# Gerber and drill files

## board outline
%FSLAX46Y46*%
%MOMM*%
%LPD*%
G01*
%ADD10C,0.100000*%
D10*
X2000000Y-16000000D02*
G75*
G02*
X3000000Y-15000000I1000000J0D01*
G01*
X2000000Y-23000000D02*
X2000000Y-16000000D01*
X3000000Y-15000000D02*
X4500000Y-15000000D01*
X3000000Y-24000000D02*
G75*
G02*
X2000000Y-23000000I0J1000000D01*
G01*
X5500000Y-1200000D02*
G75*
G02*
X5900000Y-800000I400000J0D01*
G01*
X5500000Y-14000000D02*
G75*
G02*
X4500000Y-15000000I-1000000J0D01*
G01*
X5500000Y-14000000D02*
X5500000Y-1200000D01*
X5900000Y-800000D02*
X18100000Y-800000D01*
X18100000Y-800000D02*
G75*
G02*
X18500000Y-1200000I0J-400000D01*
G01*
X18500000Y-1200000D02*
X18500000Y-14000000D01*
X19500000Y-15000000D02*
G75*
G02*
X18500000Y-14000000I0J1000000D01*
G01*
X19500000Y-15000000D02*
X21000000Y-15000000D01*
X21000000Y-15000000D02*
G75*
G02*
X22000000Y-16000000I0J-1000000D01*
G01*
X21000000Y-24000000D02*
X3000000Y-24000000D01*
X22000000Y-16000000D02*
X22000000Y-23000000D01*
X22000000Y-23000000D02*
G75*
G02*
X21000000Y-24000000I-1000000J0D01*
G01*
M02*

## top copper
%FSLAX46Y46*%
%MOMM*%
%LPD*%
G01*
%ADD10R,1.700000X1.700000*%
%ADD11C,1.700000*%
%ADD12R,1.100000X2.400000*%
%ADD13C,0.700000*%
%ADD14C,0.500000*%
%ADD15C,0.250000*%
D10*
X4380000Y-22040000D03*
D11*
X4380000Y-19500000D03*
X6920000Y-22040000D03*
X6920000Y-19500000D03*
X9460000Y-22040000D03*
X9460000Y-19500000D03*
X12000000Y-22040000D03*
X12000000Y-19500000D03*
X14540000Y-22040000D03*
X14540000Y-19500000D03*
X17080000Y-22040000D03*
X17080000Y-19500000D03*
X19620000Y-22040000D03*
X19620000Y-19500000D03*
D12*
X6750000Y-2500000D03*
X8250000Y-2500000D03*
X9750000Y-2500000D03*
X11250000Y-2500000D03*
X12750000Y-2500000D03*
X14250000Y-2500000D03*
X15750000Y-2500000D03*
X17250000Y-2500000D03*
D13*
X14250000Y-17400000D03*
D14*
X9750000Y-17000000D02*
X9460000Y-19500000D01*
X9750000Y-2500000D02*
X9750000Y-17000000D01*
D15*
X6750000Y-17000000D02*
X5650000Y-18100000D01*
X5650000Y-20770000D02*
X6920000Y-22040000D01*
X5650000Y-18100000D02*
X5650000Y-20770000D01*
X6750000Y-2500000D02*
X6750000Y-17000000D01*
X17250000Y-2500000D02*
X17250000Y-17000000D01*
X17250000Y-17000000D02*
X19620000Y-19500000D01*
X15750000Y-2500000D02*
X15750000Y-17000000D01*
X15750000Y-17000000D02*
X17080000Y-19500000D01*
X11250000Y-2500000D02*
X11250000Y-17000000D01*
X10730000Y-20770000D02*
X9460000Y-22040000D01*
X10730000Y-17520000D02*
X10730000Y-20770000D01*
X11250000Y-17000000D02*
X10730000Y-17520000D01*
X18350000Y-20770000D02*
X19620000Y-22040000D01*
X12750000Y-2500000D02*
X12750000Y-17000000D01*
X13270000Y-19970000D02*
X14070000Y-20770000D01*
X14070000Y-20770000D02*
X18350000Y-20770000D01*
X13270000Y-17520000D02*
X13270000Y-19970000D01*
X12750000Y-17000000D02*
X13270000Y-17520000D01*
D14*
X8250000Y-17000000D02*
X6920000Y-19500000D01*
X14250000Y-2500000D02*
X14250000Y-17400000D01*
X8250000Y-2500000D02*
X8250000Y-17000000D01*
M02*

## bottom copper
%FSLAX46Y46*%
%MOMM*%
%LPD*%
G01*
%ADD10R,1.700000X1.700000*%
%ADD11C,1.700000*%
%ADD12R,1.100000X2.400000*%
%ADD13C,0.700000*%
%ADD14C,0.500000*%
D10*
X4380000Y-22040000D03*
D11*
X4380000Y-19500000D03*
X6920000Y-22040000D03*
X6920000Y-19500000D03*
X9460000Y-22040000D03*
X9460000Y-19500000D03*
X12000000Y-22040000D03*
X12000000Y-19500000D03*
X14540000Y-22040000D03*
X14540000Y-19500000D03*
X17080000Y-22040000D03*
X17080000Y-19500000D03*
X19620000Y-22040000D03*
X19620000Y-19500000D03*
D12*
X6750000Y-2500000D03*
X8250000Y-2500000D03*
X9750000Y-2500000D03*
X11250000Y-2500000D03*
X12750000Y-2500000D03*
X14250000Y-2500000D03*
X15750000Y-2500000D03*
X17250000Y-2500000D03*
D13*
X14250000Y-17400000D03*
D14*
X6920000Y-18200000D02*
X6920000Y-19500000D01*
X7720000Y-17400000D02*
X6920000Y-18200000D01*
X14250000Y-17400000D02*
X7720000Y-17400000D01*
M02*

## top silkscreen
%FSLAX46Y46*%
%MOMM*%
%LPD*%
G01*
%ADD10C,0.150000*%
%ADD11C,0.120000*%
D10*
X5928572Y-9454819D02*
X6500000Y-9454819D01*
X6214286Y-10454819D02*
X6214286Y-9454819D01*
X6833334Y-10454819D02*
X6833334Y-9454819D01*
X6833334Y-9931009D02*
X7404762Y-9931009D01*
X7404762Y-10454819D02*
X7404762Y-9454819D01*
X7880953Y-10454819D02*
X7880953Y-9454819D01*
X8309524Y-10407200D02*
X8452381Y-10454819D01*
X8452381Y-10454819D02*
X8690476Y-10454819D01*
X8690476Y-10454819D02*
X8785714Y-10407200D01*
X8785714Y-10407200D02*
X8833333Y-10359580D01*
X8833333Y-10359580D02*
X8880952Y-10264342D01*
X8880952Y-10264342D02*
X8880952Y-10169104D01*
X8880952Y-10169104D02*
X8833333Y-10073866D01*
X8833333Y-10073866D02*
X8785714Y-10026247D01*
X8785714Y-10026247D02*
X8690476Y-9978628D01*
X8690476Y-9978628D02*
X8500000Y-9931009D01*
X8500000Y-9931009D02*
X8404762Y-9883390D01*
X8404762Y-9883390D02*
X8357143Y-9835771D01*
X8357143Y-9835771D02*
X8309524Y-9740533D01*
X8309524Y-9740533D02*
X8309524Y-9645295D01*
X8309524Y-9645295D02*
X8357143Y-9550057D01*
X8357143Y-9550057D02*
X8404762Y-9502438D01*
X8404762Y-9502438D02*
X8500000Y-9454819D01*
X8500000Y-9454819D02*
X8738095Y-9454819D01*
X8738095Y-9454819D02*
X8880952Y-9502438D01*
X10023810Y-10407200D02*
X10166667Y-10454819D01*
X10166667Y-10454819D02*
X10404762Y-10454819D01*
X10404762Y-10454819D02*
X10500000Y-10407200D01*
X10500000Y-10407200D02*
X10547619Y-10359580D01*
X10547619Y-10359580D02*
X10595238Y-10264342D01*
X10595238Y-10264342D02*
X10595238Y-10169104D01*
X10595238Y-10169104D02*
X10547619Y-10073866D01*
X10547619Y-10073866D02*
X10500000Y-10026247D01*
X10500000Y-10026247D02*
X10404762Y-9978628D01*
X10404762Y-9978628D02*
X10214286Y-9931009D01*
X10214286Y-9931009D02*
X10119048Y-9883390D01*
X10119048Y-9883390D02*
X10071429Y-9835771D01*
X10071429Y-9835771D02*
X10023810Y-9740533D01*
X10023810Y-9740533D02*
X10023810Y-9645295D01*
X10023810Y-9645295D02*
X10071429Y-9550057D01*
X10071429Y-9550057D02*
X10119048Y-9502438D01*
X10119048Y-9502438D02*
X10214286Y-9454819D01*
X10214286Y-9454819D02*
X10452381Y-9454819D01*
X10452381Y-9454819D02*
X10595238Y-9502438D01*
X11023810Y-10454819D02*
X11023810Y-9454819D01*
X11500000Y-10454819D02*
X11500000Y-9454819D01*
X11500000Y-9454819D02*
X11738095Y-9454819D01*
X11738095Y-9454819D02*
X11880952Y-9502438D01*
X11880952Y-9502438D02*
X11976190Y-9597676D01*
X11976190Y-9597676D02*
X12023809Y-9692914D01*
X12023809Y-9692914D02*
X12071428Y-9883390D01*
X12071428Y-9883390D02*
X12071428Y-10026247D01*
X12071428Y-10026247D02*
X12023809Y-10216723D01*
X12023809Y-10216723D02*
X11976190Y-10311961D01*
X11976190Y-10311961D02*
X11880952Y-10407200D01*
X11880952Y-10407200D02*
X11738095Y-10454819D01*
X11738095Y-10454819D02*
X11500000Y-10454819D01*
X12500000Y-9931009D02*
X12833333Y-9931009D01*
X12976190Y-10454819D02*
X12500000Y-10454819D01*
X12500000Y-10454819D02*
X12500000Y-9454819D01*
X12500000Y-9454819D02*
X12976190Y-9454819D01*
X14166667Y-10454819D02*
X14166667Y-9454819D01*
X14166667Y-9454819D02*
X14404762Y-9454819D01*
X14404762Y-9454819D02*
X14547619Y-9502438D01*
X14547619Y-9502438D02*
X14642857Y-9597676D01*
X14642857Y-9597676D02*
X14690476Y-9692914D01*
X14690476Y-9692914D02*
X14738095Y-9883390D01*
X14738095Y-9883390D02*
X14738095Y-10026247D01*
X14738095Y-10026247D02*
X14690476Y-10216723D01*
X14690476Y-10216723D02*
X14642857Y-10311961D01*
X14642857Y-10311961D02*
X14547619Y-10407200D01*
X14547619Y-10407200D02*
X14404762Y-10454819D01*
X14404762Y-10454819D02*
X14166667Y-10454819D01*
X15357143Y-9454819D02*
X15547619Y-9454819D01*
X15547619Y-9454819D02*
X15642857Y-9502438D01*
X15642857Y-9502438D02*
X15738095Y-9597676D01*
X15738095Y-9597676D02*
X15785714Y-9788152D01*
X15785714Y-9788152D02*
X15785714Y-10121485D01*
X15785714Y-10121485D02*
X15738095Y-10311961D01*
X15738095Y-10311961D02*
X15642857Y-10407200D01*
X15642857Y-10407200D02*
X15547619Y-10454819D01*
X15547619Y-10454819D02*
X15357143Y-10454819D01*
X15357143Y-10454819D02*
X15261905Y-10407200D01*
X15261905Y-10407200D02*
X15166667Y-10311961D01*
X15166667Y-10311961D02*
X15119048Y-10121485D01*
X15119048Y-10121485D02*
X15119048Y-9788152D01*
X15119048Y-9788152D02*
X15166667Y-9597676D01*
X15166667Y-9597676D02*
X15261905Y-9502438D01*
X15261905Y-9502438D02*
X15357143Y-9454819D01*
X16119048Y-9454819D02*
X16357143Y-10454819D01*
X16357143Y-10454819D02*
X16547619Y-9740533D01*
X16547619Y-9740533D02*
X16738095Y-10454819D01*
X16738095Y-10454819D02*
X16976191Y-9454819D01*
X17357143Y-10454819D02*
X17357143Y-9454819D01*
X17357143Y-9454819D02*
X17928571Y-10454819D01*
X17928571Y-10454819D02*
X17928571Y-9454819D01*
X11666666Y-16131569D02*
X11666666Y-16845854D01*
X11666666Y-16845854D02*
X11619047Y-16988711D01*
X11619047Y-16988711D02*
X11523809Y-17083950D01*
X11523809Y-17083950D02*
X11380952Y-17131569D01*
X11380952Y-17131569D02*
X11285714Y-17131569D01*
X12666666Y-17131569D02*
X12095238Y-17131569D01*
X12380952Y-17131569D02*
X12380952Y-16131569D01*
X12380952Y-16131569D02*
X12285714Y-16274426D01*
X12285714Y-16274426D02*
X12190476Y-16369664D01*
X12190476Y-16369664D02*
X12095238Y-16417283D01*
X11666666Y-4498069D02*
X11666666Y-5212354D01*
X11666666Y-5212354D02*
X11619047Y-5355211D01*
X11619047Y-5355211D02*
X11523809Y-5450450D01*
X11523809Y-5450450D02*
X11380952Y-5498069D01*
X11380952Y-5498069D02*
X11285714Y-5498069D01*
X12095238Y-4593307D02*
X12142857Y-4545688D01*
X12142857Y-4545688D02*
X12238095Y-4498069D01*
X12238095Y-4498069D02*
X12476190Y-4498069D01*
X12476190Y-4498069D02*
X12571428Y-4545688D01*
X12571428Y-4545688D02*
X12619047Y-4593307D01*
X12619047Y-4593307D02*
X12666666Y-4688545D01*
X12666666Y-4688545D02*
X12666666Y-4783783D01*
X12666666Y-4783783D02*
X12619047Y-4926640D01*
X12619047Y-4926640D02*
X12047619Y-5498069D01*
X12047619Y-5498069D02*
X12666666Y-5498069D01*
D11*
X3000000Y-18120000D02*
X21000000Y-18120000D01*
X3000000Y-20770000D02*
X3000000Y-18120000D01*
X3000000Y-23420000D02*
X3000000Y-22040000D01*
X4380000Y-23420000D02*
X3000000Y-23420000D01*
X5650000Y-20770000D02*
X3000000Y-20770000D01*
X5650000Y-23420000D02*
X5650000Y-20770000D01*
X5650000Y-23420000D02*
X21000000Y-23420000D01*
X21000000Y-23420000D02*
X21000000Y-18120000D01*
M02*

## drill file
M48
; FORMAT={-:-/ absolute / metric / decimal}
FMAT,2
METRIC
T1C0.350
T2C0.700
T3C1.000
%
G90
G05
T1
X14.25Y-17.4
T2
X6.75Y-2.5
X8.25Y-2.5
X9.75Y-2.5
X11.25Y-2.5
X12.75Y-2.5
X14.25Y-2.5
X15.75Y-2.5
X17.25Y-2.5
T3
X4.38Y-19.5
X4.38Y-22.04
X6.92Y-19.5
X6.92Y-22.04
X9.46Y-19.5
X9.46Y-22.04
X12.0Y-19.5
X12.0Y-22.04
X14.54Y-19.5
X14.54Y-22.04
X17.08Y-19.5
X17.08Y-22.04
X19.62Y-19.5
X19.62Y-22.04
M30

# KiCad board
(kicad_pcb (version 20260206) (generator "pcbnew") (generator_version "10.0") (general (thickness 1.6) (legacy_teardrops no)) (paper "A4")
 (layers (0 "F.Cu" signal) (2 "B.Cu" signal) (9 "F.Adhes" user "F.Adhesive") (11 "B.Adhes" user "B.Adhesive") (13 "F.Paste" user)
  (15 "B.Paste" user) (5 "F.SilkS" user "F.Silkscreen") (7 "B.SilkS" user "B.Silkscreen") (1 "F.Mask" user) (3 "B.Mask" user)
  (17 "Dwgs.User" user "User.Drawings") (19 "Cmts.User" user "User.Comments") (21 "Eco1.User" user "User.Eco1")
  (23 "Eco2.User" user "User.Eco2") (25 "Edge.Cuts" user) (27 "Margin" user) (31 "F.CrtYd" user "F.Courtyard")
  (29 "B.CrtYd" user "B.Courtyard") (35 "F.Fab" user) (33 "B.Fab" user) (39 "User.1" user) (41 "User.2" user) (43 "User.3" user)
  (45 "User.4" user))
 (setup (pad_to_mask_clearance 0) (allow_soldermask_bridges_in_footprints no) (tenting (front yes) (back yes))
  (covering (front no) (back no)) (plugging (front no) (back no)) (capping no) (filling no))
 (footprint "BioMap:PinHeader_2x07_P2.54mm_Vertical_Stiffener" (layer "F.Cu") (at 4.38 22.04 90)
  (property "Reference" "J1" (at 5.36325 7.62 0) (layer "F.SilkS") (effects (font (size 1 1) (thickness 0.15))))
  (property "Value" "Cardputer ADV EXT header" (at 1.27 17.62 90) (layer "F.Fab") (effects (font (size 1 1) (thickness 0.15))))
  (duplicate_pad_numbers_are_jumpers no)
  (fp_line (start 3.92 -1.38) (end 3.92 16.62) (stroke (width 0.12) (type solid)) (layer "F.SilkS"))
  (fp_line (start 1.27 -1.38) (end 3.92 -1.38) (stroke (width 0.12) (type solid)) (layer "F.SilkS"))
  (fp_line (start -1.38 -1.38) (end 0 -1.38) (stroke (width 0.12) (type solid)) (layer "F.SilkS"))
  (fp_line (start -1.38 0) (end -1.38 -1.38) (stroke (width 0.12) (type solid)) (layer "F.SilkS"))
  (fp_line (start 1.27 1.27) (end 1.27 -1.38) (stroke (width 0.12) (type solid)) (layer "F.SilkS"))
  (fp_line (start -1.38 1.27) (end 1.27 1.27) (stroke (width 0.12) (type solid)) (layer "F.SilkS"))
  (fp_line (start -1.38 1.27) (end -1.38 16.62) (stroke (width 0.12) (type solid)) (layer "F.SilkS"))
  (fp_line (start -1.38 16.62) (end 3.92 16.62) (stroke (width 0.12) (type solid)) (layer "F.SilkS"))
  (pad "1" thru_hole rect (at 0 0 90) (size 1.7 1.7) (drill 1) (layers "*.Cu" "B.Mask") (remove_unused_layers no)
   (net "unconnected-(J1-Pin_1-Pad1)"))
  (pad "2" thru_hole circle (at 2.54 0 90) (size 1.7 1.7) (drill 1) (layers "*.Cu" "B.Mask") (remove_unused_layers no)
   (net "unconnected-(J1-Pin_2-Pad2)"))
  (pad "3" thru_hole circle (at 0 2.54 90) (size 1.7 1.7) (drill 1) (layers "*.Cu" "B.Mask") (remove_unused_layers no) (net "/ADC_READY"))
  (pad "4" thru_hole circle (at 2.54 2.54 90) (size 1.7 1.7) (drill 1) (layers "*.Cu" "B.Mask") (remove_unused_layers no) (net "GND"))
  (pad "5" thru_hole circle (at 0 5.08 90) (size 1.7 1.7) (drill 1) (layers "*.Cu" "B.Mask") (remove_unused_layers no) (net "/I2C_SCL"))
  (pad "6" thru_hole circle (at 2.54 5.08 90) (size 1.7 1.7) (drill 1) (layers "*.Cu" "B.Mask") (remove_unused_layers no) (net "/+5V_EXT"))
  (pad "7" thru_hole circle (at 0 7.62 90) (size 1.7 1.7) (drill 1) (layers "*.Cu" "B.Mask") (remove_unused_layers no)
   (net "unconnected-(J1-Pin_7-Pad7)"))
  (pad "8" thru_hole circle (at 2.54 7.62 90) (size 1.7 1.7) (drill 1) (layers "*.Cu" "B.Mask") (remove_unused_layers no)
   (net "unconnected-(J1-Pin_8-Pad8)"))
  (pad "9" thru_hole circle (at 0 10.16 90) (size 1.7 1.7) (drill 1) (layers "*.Cu" "B.Mask") (remove_unused_layers no)
   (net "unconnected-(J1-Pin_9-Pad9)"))
  (pad "10" thru_hole circle (at 2.54 10.16 90) (size 1.7 1.7) (drill 1) (layers "*.Cu" "B.Mask") (remove_unused_layers no)
   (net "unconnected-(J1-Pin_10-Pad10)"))
  (pad "11" thru_hole circle (at 0 12.7 90) (size 1.7 1.7) (drill 1) (layers "*.Cu" "B.Mask") (remove_unused_layers no)
   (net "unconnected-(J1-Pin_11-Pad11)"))
  (pad "12" thru_hole circle (at 2.54 12.7 90) (size 1.7 1.7) (drill 1) (layers "*.Cu" "B.Mask") (remove_unused_layers no)
   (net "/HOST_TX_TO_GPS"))
  (pad "13" thru_hole circle (at 0 15.24 90) (size 1.7 1.7) (drill 1) (layers "*.Cu" "B.Mask") (remove_unused_layers no) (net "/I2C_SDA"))
  (pad "14" thru_hole circle (at 2.54 15.24 90) (size 1.7 1.7) (drill 1) (layers "*.Cu" "B.Mask") (remove_unused_layers no)
   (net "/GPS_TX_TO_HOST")))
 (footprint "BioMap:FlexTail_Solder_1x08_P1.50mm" (layer "F.Cu") (at 12 2.5)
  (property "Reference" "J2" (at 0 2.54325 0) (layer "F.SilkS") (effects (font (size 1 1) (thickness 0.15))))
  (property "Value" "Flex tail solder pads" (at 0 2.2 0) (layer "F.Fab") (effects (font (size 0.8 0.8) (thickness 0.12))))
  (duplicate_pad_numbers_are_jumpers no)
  (pad "1" thru_hole rect (at -5.25 0) (size 1.1 2.4) (drill 0.7) (layers "*.Cu" "*.Mask") (remove_unused_layers no) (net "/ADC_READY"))
  (pad "2" thru_hole rect (at -3.75 0) (size 1.1 2.4) (drill 0.7) (layers "*.Cu" "*.Mask") (remove_unused_layers no) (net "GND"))
  (pad "3" thru_hole rect (at -2.25 0) (size 1.1 2.4) (drill 0.7) (layers "*.Cu" "*.Mask") (remove_unused_layers no) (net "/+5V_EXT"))
  (pad "4" thru_hole rect (at -0.75 0) (size 1.1 2.4) (drill 0.7) (layers "*.Cu" "*.Mask") (remove_unused_layers no) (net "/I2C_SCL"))
  (pad "5" thru_hole rect (at 0.75 0) (size 1.1 2.4) (drill 0.7) (layers "*.Cu" "*.Mask") (remove_unused_layers no) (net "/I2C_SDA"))
  (pad "6" thru_hole rect (at 2.25 0) (size 1.1 2.4) (drill 0.7) (layers "*.Cu" "*.Mask") (remove_unused_layers no) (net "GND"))
  (pad "7" thru_hole rect (at 3.75 0) (size 1.1 2.4) (drill 0.7) (layers "*.Cu" "*.Mask") (remove_unused_layers no) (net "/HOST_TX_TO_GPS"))
  (pad "8" thru_hole rect (at 5.25 0) (size 1.1 2.4) (drill 0.7) (layers "*.Cu" "*.Mask") (remove_unused_layers no) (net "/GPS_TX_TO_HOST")))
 (gr_arc (start 2 16) (mid 2.292893 15.292893) (end 3 15) (stroke (width 0.1) (type default)) (layer "Edge.Cuts"))
 (gr_line (start 2 23) (end 2 16) (stroke (width 0.1) (type default)) (layer "Edge.Cuts"))
 (gr_line (start 3 15) (end 4.5 15) (stroke (width 0.1) (type default)) (layer "Edge.Cuts"))
 (gr_arc (start 3 24) (mid 2.292893 23.707107) (end 2 23) (stroke (width 0.1) (type default)) (layer "Edge.Cuts"))
 (gr_arc (start 5.5 1.2) (mid 5.617157 0.917157) (end 5.9 0.8) (stroke (width 0.1) (type default)) (layer "Edge.Cuts"))
 (gr_arc (start 5.5 14) (mid 5.207107 14.707107) (end 4.5 15) (stroke (width 0.1) (type default)) (layer "Edge.Cuts"))
 (gr_line (start 5.5 14) (end 5.5 1.2) (stroke (width 0.1) (type default)) (layer "Edge.Cuts"))
 (gr_line (start 5.9 0.8) (end 18.1 0.8) (stroke (width 0.1) (type default)) (layer "Edge.Cuts"))
 (gr_arc (start 18.1 0.8) (mid 18.382843 0.917157) (end 18.5 1.2) (stroke (width 0.1) (type default)) (layer "Edge.Cuts"))
 (gr_line (start 18.5 1.2) (end 18.5 14) (stroke (width 0.1) (type default)) (layer "Edge.Cuts"))
 (gr_arc (start 19.5 15) (mid 18.792893 14.707107) (end 18.5 14) (stroke (width 0.1) (type default)) (layer "Edge.Cuts"))
 (gr_line (start 19.5 15) (end 21 15) (stroke (width 0.1) (type default)) (layer "Edge.Cuts"))
 (gr_arc (start 21 15) (mid 21.707107 15.292893) (end 22 16) (stroke (width 0.1) (type default)) (layer "Edge.Cuts"))
 (gr_line (start 21 24) (end 3 24) (stroke (width 0.1) (type default)) (layer "Edge.Cuts"))
 (gr_line (start 22 16) (end 22 23) (stroke (width 0.1) (type default)) (layer "Edge.Cuts"))
 (gr_arc (start 22 23) (mid 21.707107 23.707107) (end 21 24) (stroke (width 0.1) (type default)) (layer "Edge.Cuts"))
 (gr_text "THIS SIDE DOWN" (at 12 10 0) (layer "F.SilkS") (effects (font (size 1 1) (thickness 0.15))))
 (segment (start 9.75 17) (end 9.46 19.5) (width 0.5) (layer "F.Cu") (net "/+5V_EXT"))
 (segment (start 9.75 2.5) (end 9.75 17) (width 0.5) (layer "F.Cu") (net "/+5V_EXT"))
 (segment (start 6.75 17) (end 5.65 18.1) (width 0.25) (layer "F.Cu") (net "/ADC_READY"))
 (segment (start 5.65 20.77) (end 6.92 22.04) (width 0.25) (layer "F.Cu") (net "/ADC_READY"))
 (segment (start 5.65 18.1) (end 5.65 20.77) (width 0.25) (layer "F.Cu") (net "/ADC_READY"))
 (segment (start 6.75 2.5) (end 6.75 17) (width 0.25) (layer "F.Cu") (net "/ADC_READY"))
 (segment (start 17.25 2.5) (end 17.25 17) (width 0.25) (layer "F.Cu") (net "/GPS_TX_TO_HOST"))
 (segment (start 17.25 17) (end 19.62 19.5) (width 0.25) (layer "F.Cu") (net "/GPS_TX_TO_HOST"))
 (segment (start 15.75 2.5) (end 15.75 17) (width 0.25) (layer "F.Cu") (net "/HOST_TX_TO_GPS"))
 (segment (start 15.75 17) (end 17.08 19.5) (width 0.25) (layer "F.Cu") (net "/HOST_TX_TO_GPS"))
 (segment (start 11.25 2.5) (end 11.25 17) (width 0.25) (layer "F.Cu") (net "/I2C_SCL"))
 (segment (start 10.73 20.77) (end 9.46 22.04) (width 0.25) (layer "F.Cu") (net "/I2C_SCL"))
 (segment (start 10.73 17.52) (end 10.73 20.77) (width 0.25) (layer "F.Cu") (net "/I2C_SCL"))
 (segment (start 11.25 17) (end 10.73 17.52) (width 0.25) (layer "F.Cu") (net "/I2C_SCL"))
 (segment (start 18.35 20.77) (end 19.62 22.04) (width 0.25) (layer "F.Cu") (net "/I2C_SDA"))
 (segment (start 12.75 2.5) (end 12.75 17) (width 0.25) (layer "F.Cu") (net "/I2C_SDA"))
 (segment (start 13.27 19.97) (end 14.07 20.77) (width 0.25) (layer "F.Cu") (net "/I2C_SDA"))
 (segment (start 14.07 20.77) (end 18.35 20.77) (width 0.25) (layer "F.Cu") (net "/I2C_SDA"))
 (segment (start 13.27 17.52) (end 13.27 19.97) (width 0.25) (layer "F.Cu") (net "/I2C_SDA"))
 (segment (start 12.75 17) (end 13.27 17.52) (width 0.25) (layer "F.Cu") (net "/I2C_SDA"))
 (segment (start 8.25 17) (end 6.92 19.5) (width 0.5) (layer "F.Cu") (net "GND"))
 (segment (start 14.25 2.5) (end 14.25 17.4) (width 0.5) (layer "F.Cu") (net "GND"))
 (segment (start 8.25 2.5) (end 8.25 17) (width 0.5) (layer "F.Cu") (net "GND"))
 (via (at 14.25 17.4) (size 0.7) (drill 0.35) (layers "F.Cu" "B.Cu") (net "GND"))
 (segment (start 6.92 18.2) (end 6.92 19.5) (width 0.5) (layer "B.Cu") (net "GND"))
 (segment (start 7.72 17.4) (end 6.92 18.2) (width 0.5) (layer "B.Cu") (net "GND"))
 (segment (start 14.25 17.4) (end 7.72 17.4) (width 0.5) (layer "B.Cu") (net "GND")))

